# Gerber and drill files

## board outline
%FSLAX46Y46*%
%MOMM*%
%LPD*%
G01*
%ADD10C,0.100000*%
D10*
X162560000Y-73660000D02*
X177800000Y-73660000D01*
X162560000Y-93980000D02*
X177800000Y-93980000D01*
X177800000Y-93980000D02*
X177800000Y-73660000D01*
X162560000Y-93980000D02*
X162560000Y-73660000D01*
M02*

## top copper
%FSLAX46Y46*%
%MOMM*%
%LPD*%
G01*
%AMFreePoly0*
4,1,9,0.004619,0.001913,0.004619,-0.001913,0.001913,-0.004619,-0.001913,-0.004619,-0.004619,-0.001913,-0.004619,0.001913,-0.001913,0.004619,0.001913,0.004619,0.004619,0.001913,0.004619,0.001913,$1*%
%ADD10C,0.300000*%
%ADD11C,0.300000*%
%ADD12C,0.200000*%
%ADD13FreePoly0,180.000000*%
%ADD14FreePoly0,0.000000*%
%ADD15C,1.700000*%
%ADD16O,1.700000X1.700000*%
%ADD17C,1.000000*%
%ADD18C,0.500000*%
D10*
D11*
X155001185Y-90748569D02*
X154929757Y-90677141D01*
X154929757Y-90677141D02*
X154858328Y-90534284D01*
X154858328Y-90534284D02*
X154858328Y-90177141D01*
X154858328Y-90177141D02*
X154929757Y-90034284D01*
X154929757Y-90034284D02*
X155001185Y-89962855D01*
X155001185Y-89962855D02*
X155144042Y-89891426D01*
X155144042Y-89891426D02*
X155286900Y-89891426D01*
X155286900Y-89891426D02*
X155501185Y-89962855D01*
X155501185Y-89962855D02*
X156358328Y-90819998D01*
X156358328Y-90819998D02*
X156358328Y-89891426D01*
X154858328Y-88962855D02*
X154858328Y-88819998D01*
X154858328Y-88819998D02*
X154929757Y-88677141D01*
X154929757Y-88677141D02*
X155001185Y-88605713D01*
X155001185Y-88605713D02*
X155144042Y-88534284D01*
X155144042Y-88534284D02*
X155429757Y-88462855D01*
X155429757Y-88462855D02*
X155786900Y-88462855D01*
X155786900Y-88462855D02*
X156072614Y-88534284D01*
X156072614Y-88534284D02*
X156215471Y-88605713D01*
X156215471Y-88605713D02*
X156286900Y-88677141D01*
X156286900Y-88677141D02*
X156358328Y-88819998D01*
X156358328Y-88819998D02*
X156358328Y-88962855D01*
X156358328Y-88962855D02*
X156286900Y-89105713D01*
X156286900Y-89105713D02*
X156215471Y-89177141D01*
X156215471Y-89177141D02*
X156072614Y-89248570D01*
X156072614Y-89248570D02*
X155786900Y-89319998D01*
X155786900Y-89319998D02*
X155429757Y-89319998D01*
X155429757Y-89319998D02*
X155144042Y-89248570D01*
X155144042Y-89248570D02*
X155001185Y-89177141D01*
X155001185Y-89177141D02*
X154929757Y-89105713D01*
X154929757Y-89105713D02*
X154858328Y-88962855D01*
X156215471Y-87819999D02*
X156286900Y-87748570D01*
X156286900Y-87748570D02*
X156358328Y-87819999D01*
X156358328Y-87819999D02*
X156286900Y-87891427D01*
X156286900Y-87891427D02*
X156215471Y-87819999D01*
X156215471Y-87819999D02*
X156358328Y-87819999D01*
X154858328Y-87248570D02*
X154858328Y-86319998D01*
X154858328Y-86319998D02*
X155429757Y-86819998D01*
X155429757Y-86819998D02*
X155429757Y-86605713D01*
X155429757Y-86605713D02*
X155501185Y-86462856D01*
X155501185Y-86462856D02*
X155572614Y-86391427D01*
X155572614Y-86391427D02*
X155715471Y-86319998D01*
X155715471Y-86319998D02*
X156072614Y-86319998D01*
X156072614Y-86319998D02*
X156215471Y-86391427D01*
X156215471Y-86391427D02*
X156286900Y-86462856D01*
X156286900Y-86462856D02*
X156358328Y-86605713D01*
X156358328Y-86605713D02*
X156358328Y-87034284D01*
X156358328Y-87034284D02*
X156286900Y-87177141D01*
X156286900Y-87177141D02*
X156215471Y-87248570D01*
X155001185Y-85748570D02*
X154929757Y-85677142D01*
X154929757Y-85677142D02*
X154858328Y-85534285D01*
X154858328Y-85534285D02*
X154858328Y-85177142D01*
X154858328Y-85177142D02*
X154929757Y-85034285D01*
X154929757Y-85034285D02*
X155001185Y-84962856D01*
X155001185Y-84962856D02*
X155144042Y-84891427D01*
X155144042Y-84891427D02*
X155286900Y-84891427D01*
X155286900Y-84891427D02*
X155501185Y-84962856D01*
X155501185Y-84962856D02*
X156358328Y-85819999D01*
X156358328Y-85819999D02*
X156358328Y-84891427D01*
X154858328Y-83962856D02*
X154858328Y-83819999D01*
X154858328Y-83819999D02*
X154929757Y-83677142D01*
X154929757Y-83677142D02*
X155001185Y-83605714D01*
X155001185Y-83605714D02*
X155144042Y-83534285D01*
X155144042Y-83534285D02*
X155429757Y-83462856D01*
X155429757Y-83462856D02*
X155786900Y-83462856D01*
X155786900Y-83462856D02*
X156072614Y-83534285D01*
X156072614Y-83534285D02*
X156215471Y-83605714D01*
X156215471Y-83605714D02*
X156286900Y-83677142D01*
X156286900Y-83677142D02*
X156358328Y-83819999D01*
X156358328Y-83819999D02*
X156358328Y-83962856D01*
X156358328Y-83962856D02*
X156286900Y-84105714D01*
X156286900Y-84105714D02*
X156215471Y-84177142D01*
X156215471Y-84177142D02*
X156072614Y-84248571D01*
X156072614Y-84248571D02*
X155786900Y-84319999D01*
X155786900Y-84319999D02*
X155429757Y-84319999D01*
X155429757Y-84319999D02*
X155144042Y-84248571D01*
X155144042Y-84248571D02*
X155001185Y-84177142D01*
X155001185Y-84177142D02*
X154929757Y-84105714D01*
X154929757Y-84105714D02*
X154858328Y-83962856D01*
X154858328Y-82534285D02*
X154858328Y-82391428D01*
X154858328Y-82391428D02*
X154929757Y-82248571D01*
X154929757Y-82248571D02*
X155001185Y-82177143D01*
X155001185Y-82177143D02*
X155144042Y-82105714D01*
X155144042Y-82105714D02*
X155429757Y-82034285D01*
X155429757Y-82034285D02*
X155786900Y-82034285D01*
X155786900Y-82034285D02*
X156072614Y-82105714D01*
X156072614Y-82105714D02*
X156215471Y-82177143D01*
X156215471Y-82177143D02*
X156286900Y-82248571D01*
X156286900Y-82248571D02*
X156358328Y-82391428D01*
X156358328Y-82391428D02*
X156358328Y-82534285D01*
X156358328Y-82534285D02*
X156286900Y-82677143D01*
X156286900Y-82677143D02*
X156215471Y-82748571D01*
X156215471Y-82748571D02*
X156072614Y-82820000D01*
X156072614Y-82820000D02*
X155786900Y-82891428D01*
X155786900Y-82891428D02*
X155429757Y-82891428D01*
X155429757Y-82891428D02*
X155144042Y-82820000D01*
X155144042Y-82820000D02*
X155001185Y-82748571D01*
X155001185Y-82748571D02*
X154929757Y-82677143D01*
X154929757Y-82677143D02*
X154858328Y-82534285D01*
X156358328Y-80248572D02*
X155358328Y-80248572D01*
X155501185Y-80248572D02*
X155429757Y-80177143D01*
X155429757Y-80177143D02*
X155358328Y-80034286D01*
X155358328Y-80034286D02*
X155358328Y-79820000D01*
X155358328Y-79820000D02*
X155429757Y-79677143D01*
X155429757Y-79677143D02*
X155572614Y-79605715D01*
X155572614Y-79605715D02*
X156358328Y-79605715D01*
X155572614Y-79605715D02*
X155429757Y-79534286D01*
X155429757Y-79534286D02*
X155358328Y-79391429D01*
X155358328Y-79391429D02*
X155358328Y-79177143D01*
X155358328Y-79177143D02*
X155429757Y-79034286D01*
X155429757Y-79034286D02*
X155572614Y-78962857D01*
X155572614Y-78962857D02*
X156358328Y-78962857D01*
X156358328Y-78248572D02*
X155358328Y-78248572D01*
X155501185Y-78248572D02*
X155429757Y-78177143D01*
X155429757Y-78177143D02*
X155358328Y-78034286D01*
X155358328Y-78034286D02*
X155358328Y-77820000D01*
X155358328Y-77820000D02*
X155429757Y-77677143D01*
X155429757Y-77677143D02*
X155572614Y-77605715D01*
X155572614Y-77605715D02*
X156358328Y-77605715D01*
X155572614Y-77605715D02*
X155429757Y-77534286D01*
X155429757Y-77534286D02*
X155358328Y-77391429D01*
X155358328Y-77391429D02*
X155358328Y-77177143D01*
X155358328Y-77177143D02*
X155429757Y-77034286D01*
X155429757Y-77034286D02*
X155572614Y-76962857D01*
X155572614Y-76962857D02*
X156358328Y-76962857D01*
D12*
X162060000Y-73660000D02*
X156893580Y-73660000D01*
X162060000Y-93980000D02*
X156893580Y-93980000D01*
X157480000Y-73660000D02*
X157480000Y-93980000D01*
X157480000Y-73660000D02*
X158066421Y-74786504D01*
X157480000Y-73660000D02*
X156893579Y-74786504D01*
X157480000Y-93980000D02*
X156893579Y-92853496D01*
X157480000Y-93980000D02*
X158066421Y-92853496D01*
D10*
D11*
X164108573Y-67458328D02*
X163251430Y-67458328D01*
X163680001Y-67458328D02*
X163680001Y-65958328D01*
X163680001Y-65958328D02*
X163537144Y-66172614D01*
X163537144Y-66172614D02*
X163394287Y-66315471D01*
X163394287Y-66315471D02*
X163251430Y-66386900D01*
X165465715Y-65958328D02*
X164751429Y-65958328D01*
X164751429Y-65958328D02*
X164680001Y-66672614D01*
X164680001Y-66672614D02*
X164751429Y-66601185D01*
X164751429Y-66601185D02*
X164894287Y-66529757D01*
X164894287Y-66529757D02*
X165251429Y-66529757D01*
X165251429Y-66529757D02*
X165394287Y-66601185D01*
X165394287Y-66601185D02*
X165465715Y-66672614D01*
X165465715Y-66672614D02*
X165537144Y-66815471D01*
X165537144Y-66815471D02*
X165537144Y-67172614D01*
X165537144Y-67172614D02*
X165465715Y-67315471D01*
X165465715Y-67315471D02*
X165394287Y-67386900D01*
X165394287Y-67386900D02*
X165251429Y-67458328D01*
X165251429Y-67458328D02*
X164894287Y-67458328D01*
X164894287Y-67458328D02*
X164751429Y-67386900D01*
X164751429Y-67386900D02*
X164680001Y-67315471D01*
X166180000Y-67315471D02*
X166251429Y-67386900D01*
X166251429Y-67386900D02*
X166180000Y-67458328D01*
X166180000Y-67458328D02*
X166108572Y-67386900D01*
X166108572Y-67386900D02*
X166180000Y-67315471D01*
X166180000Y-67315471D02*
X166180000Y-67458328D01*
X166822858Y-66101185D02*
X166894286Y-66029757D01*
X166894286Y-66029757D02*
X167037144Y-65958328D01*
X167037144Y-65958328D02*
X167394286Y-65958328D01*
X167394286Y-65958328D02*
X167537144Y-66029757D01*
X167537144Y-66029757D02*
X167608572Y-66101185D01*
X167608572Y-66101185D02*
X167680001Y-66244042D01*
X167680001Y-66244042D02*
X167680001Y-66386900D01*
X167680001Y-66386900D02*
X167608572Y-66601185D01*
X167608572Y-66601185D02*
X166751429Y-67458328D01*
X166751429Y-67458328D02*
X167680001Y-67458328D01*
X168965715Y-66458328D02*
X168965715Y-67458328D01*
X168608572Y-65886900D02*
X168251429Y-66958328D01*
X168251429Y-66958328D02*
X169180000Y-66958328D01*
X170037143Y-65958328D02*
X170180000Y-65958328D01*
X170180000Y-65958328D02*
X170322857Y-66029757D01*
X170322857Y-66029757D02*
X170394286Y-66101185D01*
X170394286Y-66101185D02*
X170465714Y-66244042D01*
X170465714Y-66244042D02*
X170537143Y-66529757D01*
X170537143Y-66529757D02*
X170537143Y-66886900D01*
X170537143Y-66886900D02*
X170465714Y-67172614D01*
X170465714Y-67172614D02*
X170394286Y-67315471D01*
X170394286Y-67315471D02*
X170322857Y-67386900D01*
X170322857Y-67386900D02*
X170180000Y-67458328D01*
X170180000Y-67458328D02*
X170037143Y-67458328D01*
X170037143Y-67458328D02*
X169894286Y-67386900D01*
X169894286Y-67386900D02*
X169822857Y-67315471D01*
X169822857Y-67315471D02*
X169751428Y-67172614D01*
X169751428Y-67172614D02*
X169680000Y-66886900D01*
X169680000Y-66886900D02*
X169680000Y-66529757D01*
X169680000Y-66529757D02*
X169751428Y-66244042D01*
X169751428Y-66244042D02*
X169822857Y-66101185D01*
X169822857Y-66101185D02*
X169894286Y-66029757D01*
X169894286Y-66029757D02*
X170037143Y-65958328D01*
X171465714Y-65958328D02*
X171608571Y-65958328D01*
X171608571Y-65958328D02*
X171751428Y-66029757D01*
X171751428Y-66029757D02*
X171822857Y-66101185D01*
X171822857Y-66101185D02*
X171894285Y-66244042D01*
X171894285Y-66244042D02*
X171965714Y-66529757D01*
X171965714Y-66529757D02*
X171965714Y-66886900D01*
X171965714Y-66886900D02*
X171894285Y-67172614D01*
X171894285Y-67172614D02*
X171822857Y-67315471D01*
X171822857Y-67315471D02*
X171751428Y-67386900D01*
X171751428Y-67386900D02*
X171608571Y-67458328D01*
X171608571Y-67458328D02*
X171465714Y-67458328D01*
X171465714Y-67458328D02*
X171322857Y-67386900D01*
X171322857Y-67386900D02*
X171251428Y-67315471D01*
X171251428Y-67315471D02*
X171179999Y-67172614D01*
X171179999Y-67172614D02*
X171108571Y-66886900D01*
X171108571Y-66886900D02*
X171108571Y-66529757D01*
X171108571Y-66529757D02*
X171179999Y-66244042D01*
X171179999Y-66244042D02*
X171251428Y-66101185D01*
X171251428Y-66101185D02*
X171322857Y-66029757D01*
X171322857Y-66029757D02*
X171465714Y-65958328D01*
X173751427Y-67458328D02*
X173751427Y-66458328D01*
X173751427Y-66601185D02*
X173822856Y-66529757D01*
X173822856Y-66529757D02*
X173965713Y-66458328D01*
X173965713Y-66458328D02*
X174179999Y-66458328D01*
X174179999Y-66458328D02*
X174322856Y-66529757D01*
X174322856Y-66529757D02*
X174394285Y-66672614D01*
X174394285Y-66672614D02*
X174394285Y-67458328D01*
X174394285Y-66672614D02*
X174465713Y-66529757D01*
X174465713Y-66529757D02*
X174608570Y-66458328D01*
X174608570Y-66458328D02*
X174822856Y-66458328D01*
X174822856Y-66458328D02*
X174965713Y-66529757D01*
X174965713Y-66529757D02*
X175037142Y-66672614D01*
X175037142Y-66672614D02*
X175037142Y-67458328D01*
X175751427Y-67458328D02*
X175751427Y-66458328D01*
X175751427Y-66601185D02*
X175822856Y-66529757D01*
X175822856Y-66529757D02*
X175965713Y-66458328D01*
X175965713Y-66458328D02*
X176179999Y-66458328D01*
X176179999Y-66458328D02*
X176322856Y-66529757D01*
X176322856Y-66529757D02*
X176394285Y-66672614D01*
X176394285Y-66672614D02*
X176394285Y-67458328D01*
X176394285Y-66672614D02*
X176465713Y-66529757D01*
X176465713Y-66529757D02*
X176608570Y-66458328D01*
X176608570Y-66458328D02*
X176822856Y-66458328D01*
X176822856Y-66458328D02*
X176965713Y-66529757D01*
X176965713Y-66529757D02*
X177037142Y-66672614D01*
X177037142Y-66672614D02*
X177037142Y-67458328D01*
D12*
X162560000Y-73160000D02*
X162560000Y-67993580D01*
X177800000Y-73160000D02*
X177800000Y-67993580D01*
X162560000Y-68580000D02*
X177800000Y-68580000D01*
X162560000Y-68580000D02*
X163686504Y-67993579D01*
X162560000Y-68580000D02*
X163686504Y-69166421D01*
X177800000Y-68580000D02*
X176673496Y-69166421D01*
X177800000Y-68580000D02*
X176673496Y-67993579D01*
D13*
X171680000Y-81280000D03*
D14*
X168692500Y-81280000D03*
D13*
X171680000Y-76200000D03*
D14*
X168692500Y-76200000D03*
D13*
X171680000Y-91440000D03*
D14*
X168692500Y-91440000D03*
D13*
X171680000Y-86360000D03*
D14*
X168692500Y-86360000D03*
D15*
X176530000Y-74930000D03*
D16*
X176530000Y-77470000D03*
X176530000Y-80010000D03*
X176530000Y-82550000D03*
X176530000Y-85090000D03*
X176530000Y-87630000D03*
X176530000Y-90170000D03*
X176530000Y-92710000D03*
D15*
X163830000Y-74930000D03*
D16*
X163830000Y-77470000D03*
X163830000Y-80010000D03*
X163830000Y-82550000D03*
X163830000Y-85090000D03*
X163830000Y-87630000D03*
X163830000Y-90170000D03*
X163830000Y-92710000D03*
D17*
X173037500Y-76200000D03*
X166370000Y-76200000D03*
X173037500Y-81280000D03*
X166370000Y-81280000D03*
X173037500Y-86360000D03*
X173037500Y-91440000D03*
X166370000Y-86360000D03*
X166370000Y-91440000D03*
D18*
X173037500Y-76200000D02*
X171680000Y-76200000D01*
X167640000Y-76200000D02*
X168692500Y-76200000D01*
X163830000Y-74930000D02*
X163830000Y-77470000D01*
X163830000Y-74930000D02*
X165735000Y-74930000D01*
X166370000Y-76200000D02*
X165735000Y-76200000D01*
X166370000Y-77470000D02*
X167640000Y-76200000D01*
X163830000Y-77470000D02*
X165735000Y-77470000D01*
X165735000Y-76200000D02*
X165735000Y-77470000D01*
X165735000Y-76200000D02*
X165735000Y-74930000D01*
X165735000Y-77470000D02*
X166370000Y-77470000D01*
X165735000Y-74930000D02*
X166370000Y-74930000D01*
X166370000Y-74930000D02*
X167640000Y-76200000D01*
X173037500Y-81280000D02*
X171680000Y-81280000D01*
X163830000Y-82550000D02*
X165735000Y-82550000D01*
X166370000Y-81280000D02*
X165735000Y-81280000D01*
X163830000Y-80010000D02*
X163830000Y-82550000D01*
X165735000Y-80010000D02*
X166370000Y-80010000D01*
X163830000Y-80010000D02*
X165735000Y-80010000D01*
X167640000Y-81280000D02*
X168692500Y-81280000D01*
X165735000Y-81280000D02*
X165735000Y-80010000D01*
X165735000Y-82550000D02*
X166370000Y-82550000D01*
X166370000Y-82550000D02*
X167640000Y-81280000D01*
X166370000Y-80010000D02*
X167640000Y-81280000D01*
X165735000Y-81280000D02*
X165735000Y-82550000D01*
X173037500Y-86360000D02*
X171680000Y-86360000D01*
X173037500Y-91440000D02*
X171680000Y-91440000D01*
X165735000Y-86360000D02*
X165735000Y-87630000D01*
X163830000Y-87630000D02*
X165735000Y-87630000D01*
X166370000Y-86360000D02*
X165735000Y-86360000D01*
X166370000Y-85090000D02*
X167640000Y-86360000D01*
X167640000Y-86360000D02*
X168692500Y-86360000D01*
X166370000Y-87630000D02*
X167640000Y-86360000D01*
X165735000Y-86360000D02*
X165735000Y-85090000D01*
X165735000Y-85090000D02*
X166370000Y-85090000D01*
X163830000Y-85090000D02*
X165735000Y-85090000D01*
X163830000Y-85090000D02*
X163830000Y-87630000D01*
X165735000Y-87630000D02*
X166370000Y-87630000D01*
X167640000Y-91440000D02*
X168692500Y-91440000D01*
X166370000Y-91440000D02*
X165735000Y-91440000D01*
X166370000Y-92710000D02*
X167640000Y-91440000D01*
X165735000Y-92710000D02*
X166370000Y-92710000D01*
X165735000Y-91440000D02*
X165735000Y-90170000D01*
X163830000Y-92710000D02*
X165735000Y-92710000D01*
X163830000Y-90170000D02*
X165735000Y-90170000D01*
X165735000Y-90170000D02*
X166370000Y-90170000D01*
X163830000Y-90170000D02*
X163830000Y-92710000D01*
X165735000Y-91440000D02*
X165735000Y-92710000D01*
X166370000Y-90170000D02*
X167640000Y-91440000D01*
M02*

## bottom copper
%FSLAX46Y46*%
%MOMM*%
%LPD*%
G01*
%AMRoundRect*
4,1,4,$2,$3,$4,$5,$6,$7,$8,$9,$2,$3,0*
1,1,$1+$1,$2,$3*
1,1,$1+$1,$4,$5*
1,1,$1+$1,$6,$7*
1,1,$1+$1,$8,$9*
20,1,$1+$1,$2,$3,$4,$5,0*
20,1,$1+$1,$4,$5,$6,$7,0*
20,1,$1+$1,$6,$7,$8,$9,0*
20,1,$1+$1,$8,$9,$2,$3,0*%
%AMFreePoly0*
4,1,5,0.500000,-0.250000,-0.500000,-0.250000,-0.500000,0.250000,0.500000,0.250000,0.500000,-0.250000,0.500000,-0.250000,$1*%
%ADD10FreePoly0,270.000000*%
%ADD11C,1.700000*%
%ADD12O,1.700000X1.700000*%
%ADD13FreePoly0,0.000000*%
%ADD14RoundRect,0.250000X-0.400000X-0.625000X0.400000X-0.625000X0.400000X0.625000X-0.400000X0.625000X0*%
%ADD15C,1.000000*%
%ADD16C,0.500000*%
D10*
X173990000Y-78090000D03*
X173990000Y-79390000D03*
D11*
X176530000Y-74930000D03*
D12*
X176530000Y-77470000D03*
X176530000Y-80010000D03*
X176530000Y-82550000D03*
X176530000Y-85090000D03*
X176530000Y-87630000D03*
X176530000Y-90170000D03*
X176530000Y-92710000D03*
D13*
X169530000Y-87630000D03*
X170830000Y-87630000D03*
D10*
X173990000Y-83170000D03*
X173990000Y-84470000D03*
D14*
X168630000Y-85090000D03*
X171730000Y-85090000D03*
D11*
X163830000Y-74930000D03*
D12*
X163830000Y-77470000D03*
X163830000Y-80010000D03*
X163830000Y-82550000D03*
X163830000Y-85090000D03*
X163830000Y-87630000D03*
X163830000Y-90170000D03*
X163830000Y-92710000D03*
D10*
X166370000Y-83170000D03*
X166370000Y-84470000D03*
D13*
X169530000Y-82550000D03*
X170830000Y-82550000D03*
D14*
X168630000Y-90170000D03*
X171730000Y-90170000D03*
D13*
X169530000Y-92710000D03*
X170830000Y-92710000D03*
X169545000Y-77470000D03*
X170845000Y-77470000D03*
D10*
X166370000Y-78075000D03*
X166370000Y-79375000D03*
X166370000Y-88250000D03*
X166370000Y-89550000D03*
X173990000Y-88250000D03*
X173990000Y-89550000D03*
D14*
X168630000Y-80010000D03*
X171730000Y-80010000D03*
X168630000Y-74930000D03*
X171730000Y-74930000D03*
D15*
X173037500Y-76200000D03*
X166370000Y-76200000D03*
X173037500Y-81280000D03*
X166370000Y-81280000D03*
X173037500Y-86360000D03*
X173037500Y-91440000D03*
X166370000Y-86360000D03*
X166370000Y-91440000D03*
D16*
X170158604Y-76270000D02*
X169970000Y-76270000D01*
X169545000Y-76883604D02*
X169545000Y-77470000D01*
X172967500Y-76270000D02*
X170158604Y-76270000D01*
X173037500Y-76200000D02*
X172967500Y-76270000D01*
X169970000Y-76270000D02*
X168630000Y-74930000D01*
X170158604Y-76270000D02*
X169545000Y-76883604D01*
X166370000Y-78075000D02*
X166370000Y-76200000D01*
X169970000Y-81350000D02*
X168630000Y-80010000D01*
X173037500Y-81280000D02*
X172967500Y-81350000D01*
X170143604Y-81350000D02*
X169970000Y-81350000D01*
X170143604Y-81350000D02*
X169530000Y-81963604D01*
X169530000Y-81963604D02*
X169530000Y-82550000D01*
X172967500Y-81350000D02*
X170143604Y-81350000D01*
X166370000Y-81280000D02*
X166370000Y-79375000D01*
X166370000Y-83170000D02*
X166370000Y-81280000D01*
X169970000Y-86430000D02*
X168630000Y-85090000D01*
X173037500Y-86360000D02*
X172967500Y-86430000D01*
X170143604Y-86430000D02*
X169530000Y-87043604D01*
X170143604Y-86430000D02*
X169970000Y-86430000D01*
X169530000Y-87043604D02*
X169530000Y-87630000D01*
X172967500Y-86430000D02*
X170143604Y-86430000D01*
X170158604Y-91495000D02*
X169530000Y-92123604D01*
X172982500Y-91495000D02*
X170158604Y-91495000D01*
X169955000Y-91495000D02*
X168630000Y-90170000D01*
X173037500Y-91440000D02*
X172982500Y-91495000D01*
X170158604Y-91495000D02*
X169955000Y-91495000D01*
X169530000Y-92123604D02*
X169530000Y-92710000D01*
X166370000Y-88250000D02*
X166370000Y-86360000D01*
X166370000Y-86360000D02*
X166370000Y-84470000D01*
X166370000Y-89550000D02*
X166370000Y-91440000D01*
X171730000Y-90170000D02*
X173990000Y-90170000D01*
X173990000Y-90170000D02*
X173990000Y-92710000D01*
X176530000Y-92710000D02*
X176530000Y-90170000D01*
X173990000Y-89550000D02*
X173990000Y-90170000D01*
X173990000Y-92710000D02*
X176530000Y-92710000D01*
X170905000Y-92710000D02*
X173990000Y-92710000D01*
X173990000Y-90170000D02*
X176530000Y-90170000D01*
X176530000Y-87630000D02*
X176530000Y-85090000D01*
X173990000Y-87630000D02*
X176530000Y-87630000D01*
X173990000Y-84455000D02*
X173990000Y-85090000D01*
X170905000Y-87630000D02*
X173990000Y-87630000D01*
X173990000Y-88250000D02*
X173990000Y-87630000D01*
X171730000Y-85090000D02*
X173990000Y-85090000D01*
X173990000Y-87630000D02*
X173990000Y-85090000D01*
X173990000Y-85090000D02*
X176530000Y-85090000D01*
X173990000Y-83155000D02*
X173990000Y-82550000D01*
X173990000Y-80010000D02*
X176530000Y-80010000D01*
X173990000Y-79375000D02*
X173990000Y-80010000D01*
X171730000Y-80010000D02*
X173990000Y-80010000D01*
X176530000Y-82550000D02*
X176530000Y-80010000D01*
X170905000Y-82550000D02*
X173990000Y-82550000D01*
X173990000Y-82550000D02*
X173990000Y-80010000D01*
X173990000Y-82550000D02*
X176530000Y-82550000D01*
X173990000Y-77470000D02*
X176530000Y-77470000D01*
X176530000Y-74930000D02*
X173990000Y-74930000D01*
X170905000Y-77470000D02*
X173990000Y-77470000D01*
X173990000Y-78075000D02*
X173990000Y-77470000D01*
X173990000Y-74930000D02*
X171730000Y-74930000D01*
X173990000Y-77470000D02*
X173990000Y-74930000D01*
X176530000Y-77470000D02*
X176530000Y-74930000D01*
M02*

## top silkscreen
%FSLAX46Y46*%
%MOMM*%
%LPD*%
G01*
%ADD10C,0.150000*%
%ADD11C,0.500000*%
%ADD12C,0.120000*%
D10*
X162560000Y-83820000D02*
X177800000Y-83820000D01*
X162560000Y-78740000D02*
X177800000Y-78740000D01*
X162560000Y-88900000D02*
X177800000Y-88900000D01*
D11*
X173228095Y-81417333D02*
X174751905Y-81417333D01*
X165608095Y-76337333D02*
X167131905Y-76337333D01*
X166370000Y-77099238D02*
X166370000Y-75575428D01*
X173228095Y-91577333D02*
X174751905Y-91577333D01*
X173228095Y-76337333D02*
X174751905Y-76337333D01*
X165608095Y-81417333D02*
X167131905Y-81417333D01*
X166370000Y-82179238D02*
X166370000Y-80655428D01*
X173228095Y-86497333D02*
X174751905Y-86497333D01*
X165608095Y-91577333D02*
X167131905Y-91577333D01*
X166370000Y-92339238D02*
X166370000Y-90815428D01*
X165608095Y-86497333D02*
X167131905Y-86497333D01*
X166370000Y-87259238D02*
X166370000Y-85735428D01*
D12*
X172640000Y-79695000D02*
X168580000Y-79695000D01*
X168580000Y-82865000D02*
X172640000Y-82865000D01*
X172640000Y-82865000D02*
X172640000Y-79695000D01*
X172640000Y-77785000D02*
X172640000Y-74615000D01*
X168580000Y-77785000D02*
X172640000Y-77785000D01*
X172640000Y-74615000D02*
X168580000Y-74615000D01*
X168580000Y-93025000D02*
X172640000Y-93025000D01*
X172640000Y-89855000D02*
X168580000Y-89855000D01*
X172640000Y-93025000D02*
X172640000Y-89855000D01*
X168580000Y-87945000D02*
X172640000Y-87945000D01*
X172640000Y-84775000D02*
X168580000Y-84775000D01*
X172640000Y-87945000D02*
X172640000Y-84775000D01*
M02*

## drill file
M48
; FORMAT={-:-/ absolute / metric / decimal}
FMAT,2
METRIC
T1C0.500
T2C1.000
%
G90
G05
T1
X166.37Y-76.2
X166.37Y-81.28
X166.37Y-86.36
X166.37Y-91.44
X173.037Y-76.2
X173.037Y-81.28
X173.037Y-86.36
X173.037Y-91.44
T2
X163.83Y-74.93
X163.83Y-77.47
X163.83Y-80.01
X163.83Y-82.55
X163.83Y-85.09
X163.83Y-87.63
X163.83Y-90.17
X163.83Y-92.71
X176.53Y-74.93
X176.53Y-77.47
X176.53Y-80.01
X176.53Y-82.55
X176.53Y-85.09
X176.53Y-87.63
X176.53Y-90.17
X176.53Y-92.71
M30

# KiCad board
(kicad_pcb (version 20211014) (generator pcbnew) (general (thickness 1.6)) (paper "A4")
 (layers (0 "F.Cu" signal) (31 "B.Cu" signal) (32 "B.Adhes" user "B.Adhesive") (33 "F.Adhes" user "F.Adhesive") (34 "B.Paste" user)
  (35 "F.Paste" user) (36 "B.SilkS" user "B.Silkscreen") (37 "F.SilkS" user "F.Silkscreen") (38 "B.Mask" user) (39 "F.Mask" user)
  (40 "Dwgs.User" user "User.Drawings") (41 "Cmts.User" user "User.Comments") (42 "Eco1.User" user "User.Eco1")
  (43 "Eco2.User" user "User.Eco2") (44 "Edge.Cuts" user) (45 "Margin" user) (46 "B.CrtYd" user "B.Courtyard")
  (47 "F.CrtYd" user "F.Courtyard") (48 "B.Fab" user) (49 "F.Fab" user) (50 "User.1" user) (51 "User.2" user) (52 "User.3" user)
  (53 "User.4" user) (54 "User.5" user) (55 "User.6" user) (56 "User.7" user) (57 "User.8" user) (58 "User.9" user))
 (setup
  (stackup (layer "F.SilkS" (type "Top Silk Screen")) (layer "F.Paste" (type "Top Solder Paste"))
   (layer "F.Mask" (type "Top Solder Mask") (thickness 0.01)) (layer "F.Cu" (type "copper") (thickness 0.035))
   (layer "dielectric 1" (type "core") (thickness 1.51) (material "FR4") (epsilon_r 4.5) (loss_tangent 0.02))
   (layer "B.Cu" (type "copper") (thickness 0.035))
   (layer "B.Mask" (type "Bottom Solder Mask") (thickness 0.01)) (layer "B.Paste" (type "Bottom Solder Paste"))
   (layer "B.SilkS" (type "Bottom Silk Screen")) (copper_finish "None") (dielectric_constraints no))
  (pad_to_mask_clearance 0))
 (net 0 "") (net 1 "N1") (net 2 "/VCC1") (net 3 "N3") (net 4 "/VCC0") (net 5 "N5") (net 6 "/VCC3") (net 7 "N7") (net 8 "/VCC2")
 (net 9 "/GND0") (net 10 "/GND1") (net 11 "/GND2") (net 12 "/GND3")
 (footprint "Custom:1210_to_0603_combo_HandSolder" (layer "F.Cu") (at 170.18 81.28 180)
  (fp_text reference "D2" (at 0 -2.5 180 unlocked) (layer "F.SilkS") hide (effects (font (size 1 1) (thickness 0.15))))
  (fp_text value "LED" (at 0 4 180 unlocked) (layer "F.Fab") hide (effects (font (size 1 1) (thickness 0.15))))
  (fp_line (start -2.46 1.585) (end 1.6 1.585) (layer "F.SilkS") (width 0.12))
  (fp_line (start 1.6 -1.585) (end -2.46 -1.585) (layer "F.SilkS") (width 0.12))
  (fp_line (start -2.46 -1.585) (end -2.46 1.585) (layer "F.SilkS") (width 0.12))
  (pad "1" smd custom (at -1.5 0 180) (size 0.01 0.01) (layers "F.Cu" "F.Paste" "F.Mask") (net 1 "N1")
   (options (clearance outline) (anchor circle)) (primitives))
  (pad "2" smd custom (at 1.4875 0) (size 0.01 0.01) (layers "F.Cu" "F.Paste" "F.Mask") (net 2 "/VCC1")
   (options (clearance outline) (anchor circle)) (primitives)))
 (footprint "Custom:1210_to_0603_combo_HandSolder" (layer "F.Cu") (at 170.18 76.2 180)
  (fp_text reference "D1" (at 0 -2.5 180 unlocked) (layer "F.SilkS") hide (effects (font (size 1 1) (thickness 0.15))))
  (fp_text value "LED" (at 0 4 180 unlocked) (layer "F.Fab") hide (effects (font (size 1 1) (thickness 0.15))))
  (fp_line (start -2.46 -1.585) (end -2.46 1.585) (layer "F.SilkS") (width 0.12))
  (fp_line (start 1.6 -1.585) (end -2.46 -1.585) (layer "F.SilkS") (width 0.12))
  (fp_line (start -2.46 1.585) (end 1.6 1.585) (layer "F.SilkS") (width 0.12))
  (pad "1" smd custom (at -1.5 0 180) (size 0.01 0.01) (layers "F.Cu" "F.Paste" "F.Mask") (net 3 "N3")
   (options (clearance outline) (anchor circle)) (primitives))
  (pad "2" smd custom (at 1.4875 0) (size 0.01 0.01) (layers "F.Cu" "F.Paste" "F.Mask") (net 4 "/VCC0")
   (options (clearance outline) (anchor circle)) (primitives)))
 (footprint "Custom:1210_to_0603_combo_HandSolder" (layer "F.Cu") (at 170.18 91.44 180)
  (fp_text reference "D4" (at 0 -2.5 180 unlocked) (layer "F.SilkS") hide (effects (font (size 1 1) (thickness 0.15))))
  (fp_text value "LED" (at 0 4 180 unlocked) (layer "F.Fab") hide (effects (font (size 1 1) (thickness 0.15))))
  (fp_line (start 1.6 -1.585) (end -2.46 -1.585) (layer "F.SilkS") (width 0.12))
  (fp_line (start -2.46 1.585) (end 1.6 1.585) (layer "F.SilkS") (width 0.12))
  (fp_line (start -2.46 -1.585) (end -2.46 1.585) (layer "F.SilkS") (width 0.12))
  (pad "1" smd custom (at -1.5 0 180) (size 0.01 0.01) (layers "F.Cu" "F.Paste" "F.Mask") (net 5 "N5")
   (options (clearance outline) (anchor circle)) (primitives))
  (pad "2" smd custom (at 1.4875 0) (size 0.01 0.01) (layers "F.Cu" "F.Paste" "F.Mask") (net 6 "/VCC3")
   (options (clearance outline) (anchor circle)) (primitives)))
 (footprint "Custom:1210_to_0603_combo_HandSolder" (layer "F.Cu") (at 170.18 86.36 180)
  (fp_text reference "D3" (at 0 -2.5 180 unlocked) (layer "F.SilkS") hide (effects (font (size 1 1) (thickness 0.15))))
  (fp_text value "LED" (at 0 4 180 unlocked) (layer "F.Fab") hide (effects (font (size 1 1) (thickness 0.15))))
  (fp_line (start 1.6 -1.585) (end -2.46 -1.585) (layer "F.SilkS") (width 0.12))
  (fp_line (start -2.46 1.585) (end 1.6 1.585) (layer "F.SilkS") (width 0.12))
  (fp_line (start -2.46 -1.585) (end -2.46 1.585) (layer "F.SilkS") (width 0.12))
  (pad "1" smd custom (at -1.5 0 180) (size 0.01 0.01) (layers "F.Cu" "F.Paste" "F.Mask") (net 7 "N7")
   (options (clearance outline) (anchor circle)) (primitives))
  (pad "2" smd custom (at 1.4875 0) (size 0.01 0.01) (layers "F.Cu" "F.Paste" "F.Mask") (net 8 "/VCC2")
   (options (clearance outline) (anchor circle)) (primitives)))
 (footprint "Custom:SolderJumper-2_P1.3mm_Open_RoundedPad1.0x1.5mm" (layer "B.Cu") (at 173.99 78.74 -90)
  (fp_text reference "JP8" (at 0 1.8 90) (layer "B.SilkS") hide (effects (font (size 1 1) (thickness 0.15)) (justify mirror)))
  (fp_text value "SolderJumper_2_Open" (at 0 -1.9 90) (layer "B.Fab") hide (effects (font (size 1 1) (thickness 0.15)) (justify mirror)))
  (pad "1" smd custom (at -0.65 0 270) (size 1 0.5) (layers "B.Cu" "B.Mask") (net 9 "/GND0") (zone_connect 2)
   (options (clearance outline) (anchor rect)) (primitives))
  (pad "2" smd custom (at 0.65 0 270) (size 1 0.5) (layers "B.Cu" "B.Mask") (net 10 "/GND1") (zone_connect 2)
   (options (clearance outline) (anchor rect)) (primitives)))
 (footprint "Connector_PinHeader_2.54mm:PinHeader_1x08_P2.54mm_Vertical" (layer "B.Cu") (at 176.53 74.93 180)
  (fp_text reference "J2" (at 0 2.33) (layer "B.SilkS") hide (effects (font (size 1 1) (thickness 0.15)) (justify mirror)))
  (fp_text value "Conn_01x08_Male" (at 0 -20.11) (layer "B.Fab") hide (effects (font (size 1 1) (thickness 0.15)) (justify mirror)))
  (pad "1" thru_hole circle (at 0 0 180) (size 1.7 1.7) (drill 1) (layers *.Cu *.Mask) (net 9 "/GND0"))
  (pad "2" thru_hole oval (at 0 -2.54 180) (size 1.7 1.7) (drill 1) (layers *.Cu *.Mask) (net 9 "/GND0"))
  (pad "3" thru_hole oval (at 0 -5.08 180) (size 1.7 1.7) (drill 1) (layers *.Cu *.Mask) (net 10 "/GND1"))
  (pad "4" thru_hole oval (at 0 -7.62 180) (size 1.7 1.7) (drill 1) (layers *.Cu *.Mask) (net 10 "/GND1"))
  (pad "5" thru_hole oval (at 0 -10.16 180) (size 1.7 1.7) (drill 1) (layers *.Cu *.Mask) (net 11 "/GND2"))
  (pad "6" thru_hole oval (at 0 -12.7 180) (size 1.7 1.7) (drill 1) (layers *.Cu *.Mask) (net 11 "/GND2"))
  (pad "7" thru_hole oval (at 0 -15.24 180) (size 1.7 1.7) (drill 1) (layers *.Cu *.Mask) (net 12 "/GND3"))
  (pad "8" thru_hole oval (at 0 -17.78 180) (size 1.7 1.7) (drill 1) (layers *.Cu *.Mask) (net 12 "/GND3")))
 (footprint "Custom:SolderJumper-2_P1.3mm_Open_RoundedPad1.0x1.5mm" (layer "B.Cu") (at 170.18 87.63)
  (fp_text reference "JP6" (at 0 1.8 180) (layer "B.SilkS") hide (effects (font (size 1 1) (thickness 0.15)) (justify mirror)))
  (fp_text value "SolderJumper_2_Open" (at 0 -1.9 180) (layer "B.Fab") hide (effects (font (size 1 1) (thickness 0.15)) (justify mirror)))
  (pad "1" smd custom (at -0.65 0) (size 1 0.5) (layers "B.Cu" "B.Mask") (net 7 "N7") (zone_connect 2)
   (options (clearance outline) (anchor rect)) (primitives))
  (pad "2" smd custom (at 0.65 0) (size 1 0.5) (layers "B.Cu" "B.Mask") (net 11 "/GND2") (zone_connect 2)
   (options (clearance outline) (anchor rect)) (primitives)))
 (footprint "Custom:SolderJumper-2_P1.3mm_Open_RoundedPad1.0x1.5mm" (layer "B.Cu") (at 173.99 83.82 -90)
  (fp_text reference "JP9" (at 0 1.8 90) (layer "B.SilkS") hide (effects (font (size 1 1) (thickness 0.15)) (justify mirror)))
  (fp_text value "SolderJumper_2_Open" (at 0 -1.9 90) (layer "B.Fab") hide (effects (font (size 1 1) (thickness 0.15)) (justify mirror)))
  (pad "1" smd custom (at -0.65 0 270) (size 1 0.5) (layers "B.Cu" "B.Mask") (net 10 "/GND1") (zone_connect 2)
   (options (clearance outline) (anchor rect)) (primitives))
  (pad "2" smd custom (at 0.65 0 270) (size 1 0.5) (layers "B.Cu" "B.Mask") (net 11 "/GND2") (zone_connect 2)
   (options (clearance outline) (anchor rect)) (primitives)))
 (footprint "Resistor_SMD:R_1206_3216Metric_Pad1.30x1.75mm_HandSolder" (layer "B.Cu") (at 170.18 85.09)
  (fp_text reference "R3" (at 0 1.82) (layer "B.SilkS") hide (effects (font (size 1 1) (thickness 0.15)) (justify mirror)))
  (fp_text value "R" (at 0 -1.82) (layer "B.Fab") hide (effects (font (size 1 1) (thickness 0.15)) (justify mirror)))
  (pad "1" smd roundrect (at -1.55 0) (size 1.3 1.75) (layers "B.Cu" "B.Paste" "B.Mask") (roundrect_rratio 0.1923076923) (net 7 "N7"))
  (pad "2" smd roundrect (at 1.55 0) (size 1.3 1.75) (layers "B.Cu" "B.Paste" "B.Mask") (roundrect_rratio 0.1923076923) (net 11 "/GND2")))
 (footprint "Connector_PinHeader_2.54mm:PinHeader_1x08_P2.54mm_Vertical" (layer "B.Cu") (at 163.83 74.93 180)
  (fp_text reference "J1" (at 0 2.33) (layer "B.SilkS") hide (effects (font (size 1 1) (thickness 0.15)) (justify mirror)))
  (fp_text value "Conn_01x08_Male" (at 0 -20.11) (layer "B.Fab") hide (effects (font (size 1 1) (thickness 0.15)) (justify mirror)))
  (pad "1" thru_hole circle (at 0 0 180) (size 1.7 1.7) (drill 1) (layers *.Cu *.Mask) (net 4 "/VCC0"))
  (pad "2" thru_hole oval (at 0 -2.54 180) (size 1.7 1.7) (drill 1) (layers *.Cu *.Mask) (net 4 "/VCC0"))
  (pad "3" thru_hole oval (at 0 -5.08 180) (size 1.7 1.7) (drill 1) (layers *.Cu *.Mask) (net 2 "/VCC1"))
  (pad "4" thru_hole oval (at 0 -7.62 180) (size 1.7 1.7) (drill 1) (layers *.Cu *.Mask) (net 2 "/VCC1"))
  (pad "5" thru_hole oval (at 0 -10.16 180) (size 1.7 1.7) (drill 1) (layers *.Cu *.Mask) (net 8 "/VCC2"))
  (pad "6" thru_hole oval (at 0 -12.7 180) (size 1.7 1.7) (drill 1) (layers *.Cu *.Mask) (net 8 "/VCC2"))
  (pad "7" thru_hole oval (at 0 -15.24 180) (size 1.7 1.7) (drill 1) (layers *.Cu *.Mask) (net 6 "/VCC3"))
  (pad "8" thru_hole oval (at 0 -17.78 180) (size 1.7 1.7) (drill 1) (layers *.Cu *.Mask) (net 6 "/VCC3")))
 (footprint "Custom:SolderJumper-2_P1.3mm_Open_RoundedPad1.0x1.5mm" (layer "B.Cu") (at 166.37 83.82 -90)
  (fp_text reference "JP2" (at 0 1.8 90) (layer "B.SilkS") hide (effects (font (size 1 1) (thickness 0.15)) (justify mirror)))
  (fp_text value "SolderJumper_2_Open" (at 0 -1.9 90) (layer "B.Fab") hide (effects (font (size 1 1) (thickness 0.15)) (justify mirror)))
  (pad "1" smd custom (at -0.65 0 270) (size 1 0.5) (layers "B.Cu" "B.Mask") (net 2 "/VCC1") (zone_connect 2)
   (options (clearance outline) (anchor rect)) (primitives))
  (pad "2" smd custom (at 0.65 0 270) (size 1 0.5) (layers "B.Cu" "B.Mask") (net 8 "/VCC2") (zone_connect 2)
   (options (clearance outline) (anchor rect)) (primitives)))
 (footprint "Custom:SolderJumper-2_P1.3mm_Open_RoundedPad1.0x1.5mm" (layer "B.Cu") (at 170.18 82.55)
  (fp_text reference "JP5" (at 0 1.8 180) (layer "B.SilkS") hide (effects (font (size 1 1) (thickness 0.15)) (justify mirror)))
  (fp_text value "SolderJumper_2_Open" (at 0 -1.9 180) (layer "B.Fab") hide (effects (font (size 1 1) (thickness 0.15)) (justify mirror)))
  (pad "1" smd custom (at -0.65 0) (size 1 0.5) (layers "B.Cu" "B.Mask") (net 1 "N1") (zone_connect 2)
   (options (clearance outline) (anchor rect)) (primitives))
  (pad "2" smd custom (at 0.65 0) (size 1 0.5) (layers "B.Cu" "B.Mask") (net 10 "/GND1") (zone_connect 2)
   (options (clearance outline) (anchor rect)) (primitives)))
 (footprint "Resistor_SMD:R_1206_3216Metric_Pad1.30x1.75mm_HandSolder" (layer "B.Cu") (at 170.18 90.17)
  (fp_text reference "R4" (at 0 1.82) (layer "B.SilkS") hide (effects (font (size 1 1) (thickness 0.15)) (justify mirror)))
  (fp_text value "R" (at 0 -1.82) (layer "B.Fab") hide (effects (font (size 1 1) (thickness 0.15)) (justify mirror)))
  (pad "1" smd roundrect (at -1.55 0) (size 1.3 1.75) (layers "B.Cu" "B.Paste" "B.Mask") (roundrect_rratio 0.1923076923) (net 5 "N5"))
  (pad "2" smd roundrect (at 1.55 0) (size 1.3 1.75) (layers "B.Cu" "B.Paste" "B.Mask") (roundrect_rratio 0.1923076923) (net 12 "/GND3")))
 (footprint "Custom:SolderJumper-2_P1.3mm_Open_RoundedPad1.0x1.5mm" (layer "B.Cu") (at 170.18 92.71)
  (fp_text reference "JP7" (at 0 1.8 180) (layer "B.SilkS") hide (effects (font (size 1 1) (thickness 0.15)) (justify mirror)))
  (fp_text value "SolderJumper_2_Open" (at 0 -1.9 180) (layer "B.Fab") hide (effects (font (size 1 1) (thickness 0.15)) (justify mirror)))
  (pad "1" smd custom (at -0.65 0) (size 1 0.5) (layers "B.Cu" "B.Mask") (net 5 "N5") (zone_connect 2)
   (options (clearance outline) (anchor rect)) (primitives))
  (pad "2" smd custom (at 0.65 0) (size 1 0.5) (layers "B.Cu" "B.Mask") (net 12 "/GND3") (zone_connect 2)
   (options (clearance outline) (anchor rect)) (primitives)))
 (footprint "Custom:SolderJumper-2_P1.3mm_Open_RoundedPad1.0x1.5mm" (layer "B.Cu") (at 170.195 77.47)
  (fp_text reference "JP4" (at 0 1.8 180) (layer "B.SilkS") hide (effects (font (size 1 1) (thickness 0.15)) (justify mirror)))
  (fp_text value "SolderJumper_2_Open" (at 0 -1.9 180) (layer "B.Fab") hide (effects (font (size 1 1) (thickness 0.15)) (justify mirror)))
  (pad "1" smd custom (at -0.65 0) (size 1 0.5) (layers "B.Cu" "B.Mask") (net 3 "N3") (zone_connect 2)
   (options (clearance outline) (anchor rect)) (primitives))
  (pad "2" smd custom (at 0.65 0) (size 1 0.5) (layers "B.Cu" "B.Mask") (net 9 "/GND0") (zone_connect 2)
   (options (clearance outline) (anchor rect)) (primitives)))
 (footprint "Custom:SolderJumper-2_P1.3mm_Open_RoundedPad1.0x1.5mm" (layer "B.Cu") (at 166.37 78.725 -90)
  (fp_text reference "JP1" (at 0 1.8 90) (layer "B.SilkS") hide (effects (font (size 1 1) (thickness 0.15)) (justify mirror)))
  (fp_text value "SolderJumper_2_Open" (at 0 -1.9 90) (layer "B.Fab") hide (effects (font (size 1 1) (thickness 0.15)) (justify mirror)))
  (pad "1" smd custom (at -0.65 0 270) (size 1 0.5) (layers "B.Cu" "B.Mask") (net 4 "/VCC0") (zone_connect 2)
   (options (clearance outline) (anchor rect)) (primitives))
  (pad "2" smd custom (at 0.65 0 270) (size 1 0.5) (layers "B.Cu" "B.Mask") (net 2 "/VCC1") (zone_connect 2)
   (options (clearance outline) (anchor rect)) (primitives)))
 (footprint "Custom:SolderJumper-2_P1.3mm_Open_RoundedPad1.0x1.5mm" (layer "B.Cu") (at 166.37 88.9 -90)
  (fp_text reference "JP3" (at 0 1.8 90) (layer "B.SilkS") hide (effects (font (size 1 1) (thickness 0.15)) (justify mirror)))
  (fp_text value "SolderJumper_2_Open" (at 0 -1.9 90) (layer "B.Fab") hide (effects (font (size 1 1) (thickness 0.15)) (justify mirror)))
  (pad "1" smd custom (at -0.65 0 270) (size 1 0.5) (layers "B.Cu" "B.Mask") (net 8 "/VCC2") (zone_connect 2)
   (options (clearance outline) (anchor rect)) (primitives))
  (pad "2" smd custom (at 0.65 0 270) (size 1 0.5) (layers "B.Cu" "B.Mask") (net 6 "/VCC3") (zone_connect 2)
   (options (clearance outline) (anchor rect)) (primitives)))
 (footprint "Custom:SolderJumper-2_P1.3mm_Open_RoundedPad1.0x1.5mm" (layer "B.Cu") (at 173.99 88.9 -90)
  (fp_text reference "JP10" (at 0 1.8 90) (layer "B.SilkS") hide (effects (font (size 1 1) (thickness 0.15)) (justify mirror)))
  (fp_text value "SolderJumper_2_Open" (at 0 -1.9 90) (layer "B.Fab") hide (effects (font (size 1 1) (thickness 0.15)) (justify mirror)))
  (pad "1" smd custom (at -0.65 0 270) (size 1 0.5) (layers "B.Cu" "B.Mask") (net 11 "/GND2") (zone_connect 2)
   (options (clearance outline) (anchor rect)) (primitives))
  (pad "2" smd custom (at 0.65 0 270) (size 1 0.5) (layers "B.Cu" "B.Mask") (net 12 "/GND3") (zone_connect 2)
   (options (clearance outline) (anchor rect)) (primitives)))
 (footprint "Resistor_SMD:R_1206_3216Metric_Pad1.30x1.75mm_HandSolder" (layer "B.Cu") (at 170.18 80.01)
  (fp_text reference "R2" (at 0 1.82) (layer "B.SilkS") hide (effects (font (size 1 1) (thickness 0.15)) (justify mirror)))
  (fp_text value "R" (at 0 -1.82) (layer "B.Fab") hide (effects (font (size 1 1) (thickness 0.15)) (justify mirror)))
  (pad "1" smd roundrect (at -1.55 0) (size 1.3 1.75) (layers "B.Cu" "B.Paste" "B.Mask") (roundrect_rratio 0.1923076923) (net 1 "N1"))
  (pad "2" smd roundrect (at 1.55 0) (size 1.3 1.75) (layers "B.Cu" "B.Paste" "B.Mask") (roundrect_rratio 0.1923076923) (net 10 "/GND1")))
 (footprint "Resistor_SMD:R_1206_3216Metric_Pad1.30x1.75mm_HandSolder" (layer "B.Cu") (at 170.18 74.93)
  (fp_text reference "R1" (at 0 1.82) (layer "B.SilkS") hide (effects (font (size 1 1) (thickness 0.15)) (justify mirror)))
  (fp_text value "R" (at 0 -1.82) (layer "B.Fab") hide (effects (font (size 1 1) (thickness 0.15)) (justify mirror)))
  (pad "1" smd roundrect (at -1.55 0) (size 1.3 1.75) (layers "B.Cu" "B.Paste" "B.Mask") (roundrect_rratio 0.1923076923) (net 3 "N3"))
  (pad "2" smd roundrect (at 1.55 0) (size 1.3 1.75) (layers "B.Cu" "B.Paste" "B.Mask") (roundrect_rratio 0.1923076923) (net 9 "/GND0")))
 (gr_line (start 162.56 83.82) (end 177.8 83.82) (layer "F.SilkS") (width 0.15))
 (gr_line (start 162.56 78.74) (end 177.8 78.74) (layer "F.SilkS") (width 0.15))
 (gr_line (start 162.56 88.9) (end 177.8 88.9) (layer "F.SilkS") (width 0.15))
 (gr_line (start 162.56 73.66) (end 177.8 73.66) (layer "Edge.Cuts") (width 0.1))
 (gr_line (start 162.56 93.98) (end 177.8 93.98) (layer "Edge.Cuts") (width 0.1))
 (gr_line (start 177.8 93.98) (end 177.8 73.66) (layer "Edge.Cuts") (width 0.1))
 (gr_line (start 162.56 93.98) (end 162.56 73.66) (layer "Edge.Cuts") (width 0.1))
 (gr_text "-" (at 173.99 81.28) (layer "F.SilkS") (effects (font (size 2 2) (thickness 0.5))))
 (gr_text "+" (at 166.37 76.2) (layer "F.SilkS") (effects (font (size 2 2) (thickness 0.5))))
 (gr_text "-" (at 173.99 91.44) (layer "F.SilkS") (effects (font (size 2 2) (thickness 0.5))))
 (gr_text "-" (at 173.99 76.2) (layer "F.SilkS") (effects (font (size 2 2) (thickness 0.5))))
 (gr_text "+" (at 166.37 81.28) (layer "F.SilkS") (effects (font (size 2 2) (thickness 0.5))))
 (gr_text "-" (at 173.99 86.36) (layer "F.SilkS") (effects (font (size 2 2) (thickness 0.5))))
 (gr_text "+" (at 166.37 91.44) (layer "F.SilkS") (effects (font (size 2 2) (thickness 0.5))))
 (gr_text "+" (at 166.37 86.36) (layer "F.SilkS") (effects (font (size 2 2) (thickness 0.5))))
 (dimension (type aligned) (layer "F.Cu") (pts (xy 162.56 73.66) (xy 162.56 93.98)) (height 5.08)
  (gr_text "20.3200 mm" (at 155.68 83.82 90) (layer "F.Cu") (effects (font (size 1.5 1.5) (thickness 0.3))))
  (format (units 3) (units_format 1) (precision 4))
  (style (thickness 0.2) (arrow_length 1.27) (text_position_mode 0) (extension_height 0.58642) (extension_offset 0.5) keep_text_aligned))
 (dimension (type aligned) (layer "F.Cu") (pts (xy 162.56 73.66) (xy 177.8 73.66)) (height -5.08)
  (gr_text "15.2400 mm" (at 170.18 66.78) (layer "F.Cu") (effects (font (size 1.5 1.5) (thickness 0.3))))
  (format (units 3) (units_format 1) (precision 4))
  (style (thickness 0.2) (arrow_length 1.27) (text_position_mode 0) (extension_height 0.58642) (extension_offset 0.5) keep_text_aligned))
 (segment (start 173.0375 76.2) (end 171.68 76.2) (width 0.5) (layer "F.Cu") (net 3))
 (via (at 173.0375 76.2) (size 1) (drill 0.5) (layers "F.Cu" "B.Cu") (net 3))
 (segment (start 170.158604 76.27) (end 169.97 76.27) (width 0.5) (layer "B.Cu") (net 3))
 (segment (start 169.545 76.883604) (end 169.545 77.47) (width 0.5) (layer "B.Cu") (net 3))
 (segment (start 172.9675 76.27) (end 170.158604 76.27) (width 0.5) (layer "B.Cu") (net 3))
 (segment (start 173.0375 76.2) (end 172.9675 76.27) (width 0.5) (layer "B.Cu") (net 3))
 (segment (start 169.97 76.27) (end 168.63 74.93) (width 0.5) (layer "B.Cu") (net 3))
 (segment (start 170.158604 76.27) (end 169.545 76.883604) (width 0.5) (layer "B.Cu") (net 3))
 (segment (start 167.64 76.2) (end 168.6925 76.2) (width 0.5) (layer "F.Cu") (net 4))
 (segment (start 163.83 74.93) (end 163.83 77.47) (width 0.5) (layer "F.Cu") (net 4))
 (segment (start 163.83 74.93) (end 165.735 74.93) (width 0.5) (layer "F.Cu") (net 4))
 (segment (start 166.37 76.2) (end 165.735 76.2) (width 0.5) (layer "F.Cu") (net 4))
 (segment (start 166.37 77.47) (end 167.64 76.2) (width 0.5) (layer "F.Cu") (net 4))
 (segment (start 163.83 77.47) (end 165.735 77.47) (width 0.5) (layer "F.Cu") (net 4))
 (segment (start 165.735 76.2) (end 165.735 77.47) (width 0.5) (layer "F.Cu") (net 4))
 (segment (start 165.735 76.2) (end 165.735 74.93) (width 0.5) (layer "F.Cu") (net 4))
 (segment (start 165.735 77.47) (end 166.37 77.47) (width 0.5) (layer "F.Cu") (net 4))
 (segment (start 165.735 74.93) (end 166.37 74.93) (width 0.5) (layer "F.Cu") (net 4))
 (segment (start 166.37 74.93) (end 167.64 76.2) (width 0.5) (layer "F.Cu") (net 4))
 (via (at 166.37 76.2) (size 1) (drill 0.5) (layers "F.Cu" "B.Cu") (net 4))
 (segment (start 166.37 78.075) (end 166.37 76.2) (width 0.5) (layer "B.Cu") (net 4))
 (segment (start 173.0375 81.28) (end 171.68 81.28) (width 0.5) (layer "F.Cu") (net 1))
 (via (at 173.0375 81.28) (size 1) (drill 0.5) (layers "F.Cu" "B.Cu") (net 1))
 (segment (start 169.97 81.35) (end 168.63 80.01) (width 0.5) (layer "B.Cu") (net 1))
 (segment (start 173.0375 81.28) (end 172.9675 81.35) (width 0.5) (layer "B.Cu") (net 1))
 (segment (start 170.143604 81.35) (end 169.97 81.35) (width 0.5) (layer "B.Cu") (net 1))
 (segment (start 170.143604 81.35) (end 169.53 81.963604) (width 0.5) (layer "B.Cu") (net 1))
 (segment (start 169.53 81.963604) (end 169.53 82.55) (width 0.5) (layer "B.Cu") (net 1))
 (segment (start 172.9675 81.35) (end 170.143604 81.35) (width 0.5) (layer "B.Cu") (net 1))
 (segment (start 163.83 82.55) (end 165.735 82.55) (width 0.5) (layer "F.Cu") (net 2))
 (segment (start 166.37 81.28) (end 165.735 81.28) (width 0.5) (layer "F.Cu") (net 2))
 (segment (start 163.83 80.01) (end 163.83 82.55) (width 0.5) (layer "F.Cu") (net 2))
 (segment (start 165.735 80.01) (end 166.37 80.01) (width 0.5) (layer "F.Cu") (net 2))
 (segment (start 163.83 80.01) (end 165.735 80.01) (width 0.5) (layer "F.Cu") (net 2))
 (segment (start 167.64 81.28) (end 168.6925 81.28) (width 0.5) (layer "F.Cu") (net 2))
 (segment (start 165.735 81.28) (end 165.735 80.01) (width 0.5) (layer "F.Cu") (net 2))
 (segment (start 165.735 82.55) (end 166.37 82.55) (width 0.5) (layer "F.Cu") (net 2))
 (segment (start 166.37 82.55) (end 167.64 81.28) (width 0.5) (layer "F.Cu") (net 2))
 (segment (start 166.37 80.01) (end 167.64 81.28) (width 0.5) (layer "F.Cu") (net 2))
 (segment (start 165.735 81.28) (end 165.735 82.55) (width 0.5) (layer "F.Cu") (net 2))
 (via (at 166.37 81.28) (size 1) (drill 0.5) (layers "F.Cu" "B.Cu") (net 2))
 (segment (start 166.37 81.28) (end 166.37 79.375) (width 0.5) (layer "B.Cu") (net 2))
 (segment (start 166.37 83.17) (end 166.37 81.28) (width 0.5) (layer "B.Cu") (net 2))
 (segment (start 173.0375 86.36) (end 171.68 86.36) (width 0.5) (layer "F.Cu") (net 7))
 (via (at 173.0375 86.36) (size 1) (drill 0.5) (layers "F.Cu" "B.Cu") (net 7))
 (segment (start 169.97 86.43) (end 168.63 85.09) (width 0.5) (layer "B.Cu") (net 7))
 (segment (start 173.0375 86.36) (end 172.9675 86.43) (width 0.5) (layer "B.Cu") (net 7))
 (segment (start 170.143604 86.43) (end 169.53 87.043604) (width 0.5) (layer "B.Cu") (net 7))
 (segment (start 170.143604 86.43) (end 169.97 86.43) (width 0.5) (layer "B.Cu") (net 7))
 (segment (start 169.53 87.043604) (end 169.53 87.63) (width 0.5) (layer "B.Cu") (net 7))
 (segment (start 172.9675 86.43) (end 170.143604 86.43) (width 0.5) (layer "B.Cu") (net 7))
 (segment (start 173.0375 91.44) (end 171.68 91.44) (width 0.5) (layer "F.Cu") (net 5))
 (via (at 173.0375 91.44) (size 1) (drill 0.5) (layers "F.Cu" "B.Cu") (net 5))
 (segment (start 170.158604 91.495) (end 169.53 92.123604) (width 0.5) (layer "B.Cu") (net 5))
 (segment (start 172.9825 91.495) (end 170.158604 91.495) (width 0.5) (layer "B.Cu") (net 5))
 (segment (start 169.955 91.495) (end 168.63 90.17) (width 0.5) (layer "B.Cu") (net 5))
 (segment (start 173.0375 91.44) (end 172.9825 91.495) (width 0.5) (layer "B.Cu") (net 5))
 (segment (start 170.158604 91.495) (end 169.955 91.495) (width 0.5) (layer "B.Cu") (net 5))
 (segment (start 169.53 92.123604) (end 169.53 92.71) (width 0.5) (layer "B.Cu") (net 5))
 (segment (start 165.735 86.36) (end 165.735 87.63) (width 0.5) (layer "F.Cu") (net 8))
 (segment (start 163.83 87.63) (end 165.735 87.63) (width 0.5) (layer "F.Cu") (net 8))
 (segment (start 166.37 86.36) (end 165.735 86.36) (width 0.5) (layer "F.Cu") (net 8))
 (segment (start 166.37 85.09) (end 167.64 86.36) (width 0.5) (layer "F.Cu") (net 8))
 (segment (start 167.64 86.36) (end 168.6925 86.36) (width 0.5) (layer "F.Cu") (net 8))
 (segment (start 166.37 87.63) (end 167.64 86.36) (width 0.5) (layer "F.Cu") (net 8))
 (segment (start 165.735 86.36) (end 165.735 85.09) (width 0.5) (layer "F.Cu") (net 8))
 (segment (start 165.735 85.09) (end 166.37 85.09) (width 0.5) (layer "F.Cu") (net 8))
 (segment (start 163.83 85.09) (end 165.735 85.09) (width 0.5) (layer "F.Cu") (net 8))
 (segment (start 163.83 85.09) (end 163.83 87.63) (width 0.5) (layer "F.Cu") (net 8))
 (segment (start 165.735 87.63) (end 166.37 87.63) (width 0.5) (layer "F.Cu") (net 8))
 (via (at 166.37 86.36) (size 1) (drill 0.5) (layers "F.Cu" "B.Cu") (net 8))
 (segment (start 166.37 88.25) (end 166.37 86.36) (width 0.5) (layer "B.Cu") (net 8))
 (segment (start 166.37 86.36) (end 166.37 84.47) (width 0.5) (layer "B.Cu") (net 8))
 (segment (start 167.64 91.44) (end 168.6925 91.44) (width 0.5) (layer "F.Cu") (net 6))
 (segment (start 166.37 91.44) (end 165.735 91.44) (width 0.5) (layer "F.Cu") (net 6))
 (segment (start 166.37 92.71) (end 167.64 91.44) (width 0.5) (layer "F.Cu") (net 6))
 (segment (start 165.735 92.71) (end 166.37 92.71) (width 0.5) (layer "F.Cu") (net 6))
 (segment (start 165.735 91.44) (end 165.735 90.17) (width 0.5) (layer "F.Cu") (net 6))
 (segment (start 163.83 92.71) (end 165.735 92.71) (width 0.5) (layer "F.Cu") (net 6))
 (segment (start 163.83 90.17) (end 165.735 90.17) (width 0.5) (layer "F.Cu") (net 6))
 (segment (start 165.735 90.17) (end 166.37 90.17) (width 0.5) (layer "F.Cu") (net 6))
 (segment (start 163.83 90.17) (end 163.83 92.71) (width 0.5) (layer "F.Cu") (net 6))
 (segment (start 165.735 91.44) (end 165.735 92.71) (width 0.5) (layer "F.Cu") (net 6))
 (segment (start 166.37 90.17) (end 167.64 91.44) (width 0.5) (layer "F.Cu") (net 6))
 (via (at 166.37 91.44) (size 1) (drill 0.5) (layers "F.Cu" "B.Cu") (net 6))
 (segment (start 166.37 89.55) (end 166.37 91.44) (width 0.5) (layer "B.Cu") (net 6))
 (segment (start 171.73 90.17) (end 173.99 90.17) (width 0.5) (layer "B.Cu") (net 12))
 (segment (start 173.99 90.17) (end 173.99 92.71) (width 0.5) (layer "B.Cu") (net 12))
 (segment (start 176.53 92.71) (end 176.53 90.17) (width 0.5) (layer "B.Cu") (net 12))
 (segment (start 173.99 89.55) (end 173.99 90.17) (width 0.5) (layer "B.Cu") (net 12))
 (segment (start 173.99 92.71) (end 176.53 92.71) (width 0.5) (layer "B.Cu") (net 12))
 (segment (start 170.905 92.71) (end 173.99 92.71) (width 0.5) (layer "B.Cu") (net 12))
 (segment (start 173.99 90.17) (end 176.53 90.17) (width 0.5) (layer "B.Cu") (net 12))
 (segment (start 176.53 87.63) (end 176.53 85.09) (width 0.5) (layer "B.Cu") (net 11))
 (segment (start 173.99 87.63) (end 176.53 87.63) (width 0.5) (layer "B.Cu") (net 11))
 (segment (start 173.99 84.455) (end 173.99 85.09) (width 0.5) (layer "B.Cu") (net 11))
 (segment (start 170.905 87.63) (end 173.99 87.63) (width 0.5) (layer "B.Cu") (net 11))
 (segment (start 173.99 88.25) (end 173.99 87.63) (width 0.5) (layer "B.Cu") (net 11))
 (segment (start 171.73 85.09) (end 173.99 85.09) (width 0.5) (layer "B.Cu") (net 11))
 (segment (start 173.99 87.63) (end 173.99 85.09) (width 0.5) (layer "B.Cu") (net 11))
 (segment (start 173.99 85.09) (end 176.53 85.09) (width 0.5) (layer "B.Cu") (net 11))
 (segment (start 173.99 83.155) (end 173.99 82.55) (width 0.5) (layer "B.Cu") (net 10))
 (segment (start 173.99 80.01) (end 176.53 80.01) (width 0.5) (layer "B.Cu") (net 10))
 (segment (start 173.99 79.375) (end 173.99 80.01) (width 0.5) (layer "B.Cu") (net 10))
 (segment (start 171.73 80.01) (end 173.99 80.01) (width 0.5) (layer "B.Cu") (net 10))
 (segment (start 176.53 82.55) (end 176.53 80.01) (width 0.5) (layer "B.Cu") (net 10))
 (segment (start 170.905 82.55) (end 173.99 82.55) (width 0.5) (layer "B.Cu") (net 10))
 (segment (start 173.99 82.55) (end 173.99 80.01) (width 0.5) (layer "B.Cu") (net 10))
 (segment (start 173.99 82.55) (end 176.53 82.55) (width 0.5) (layer "B.Cu") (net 10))
 (segment (start 173.99 77.47) (end 176.53 77.47) (width 0.5) (layer "B.Cu") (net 9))
 (segment (start 176.53 74.93) (end 173.99 74.93) (width 0.5) (layer "B.Cu") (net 9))
 (segment (start 170.905 77.47) (end 173.99 77.47) (width 0.5) (layer "B.Cu") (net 9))
 (segment (start 173.99 78.075) (end 173.99 77.47) (width 0.5) (layer "B.Cu") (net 9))
 (segment (start 173.99 74.93) (end 171.73 74.93) (width 0.5) (layer "B.Cu") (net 9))
 (segment (start 173.99 77.47) (end 173.99 74.93) (width 0.5) (layer "B.Cu") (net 9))
 (segment (start 176.53 77.47) (end 176.53 74.93) (width 0.5) (layer "B.Cu") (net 9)))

